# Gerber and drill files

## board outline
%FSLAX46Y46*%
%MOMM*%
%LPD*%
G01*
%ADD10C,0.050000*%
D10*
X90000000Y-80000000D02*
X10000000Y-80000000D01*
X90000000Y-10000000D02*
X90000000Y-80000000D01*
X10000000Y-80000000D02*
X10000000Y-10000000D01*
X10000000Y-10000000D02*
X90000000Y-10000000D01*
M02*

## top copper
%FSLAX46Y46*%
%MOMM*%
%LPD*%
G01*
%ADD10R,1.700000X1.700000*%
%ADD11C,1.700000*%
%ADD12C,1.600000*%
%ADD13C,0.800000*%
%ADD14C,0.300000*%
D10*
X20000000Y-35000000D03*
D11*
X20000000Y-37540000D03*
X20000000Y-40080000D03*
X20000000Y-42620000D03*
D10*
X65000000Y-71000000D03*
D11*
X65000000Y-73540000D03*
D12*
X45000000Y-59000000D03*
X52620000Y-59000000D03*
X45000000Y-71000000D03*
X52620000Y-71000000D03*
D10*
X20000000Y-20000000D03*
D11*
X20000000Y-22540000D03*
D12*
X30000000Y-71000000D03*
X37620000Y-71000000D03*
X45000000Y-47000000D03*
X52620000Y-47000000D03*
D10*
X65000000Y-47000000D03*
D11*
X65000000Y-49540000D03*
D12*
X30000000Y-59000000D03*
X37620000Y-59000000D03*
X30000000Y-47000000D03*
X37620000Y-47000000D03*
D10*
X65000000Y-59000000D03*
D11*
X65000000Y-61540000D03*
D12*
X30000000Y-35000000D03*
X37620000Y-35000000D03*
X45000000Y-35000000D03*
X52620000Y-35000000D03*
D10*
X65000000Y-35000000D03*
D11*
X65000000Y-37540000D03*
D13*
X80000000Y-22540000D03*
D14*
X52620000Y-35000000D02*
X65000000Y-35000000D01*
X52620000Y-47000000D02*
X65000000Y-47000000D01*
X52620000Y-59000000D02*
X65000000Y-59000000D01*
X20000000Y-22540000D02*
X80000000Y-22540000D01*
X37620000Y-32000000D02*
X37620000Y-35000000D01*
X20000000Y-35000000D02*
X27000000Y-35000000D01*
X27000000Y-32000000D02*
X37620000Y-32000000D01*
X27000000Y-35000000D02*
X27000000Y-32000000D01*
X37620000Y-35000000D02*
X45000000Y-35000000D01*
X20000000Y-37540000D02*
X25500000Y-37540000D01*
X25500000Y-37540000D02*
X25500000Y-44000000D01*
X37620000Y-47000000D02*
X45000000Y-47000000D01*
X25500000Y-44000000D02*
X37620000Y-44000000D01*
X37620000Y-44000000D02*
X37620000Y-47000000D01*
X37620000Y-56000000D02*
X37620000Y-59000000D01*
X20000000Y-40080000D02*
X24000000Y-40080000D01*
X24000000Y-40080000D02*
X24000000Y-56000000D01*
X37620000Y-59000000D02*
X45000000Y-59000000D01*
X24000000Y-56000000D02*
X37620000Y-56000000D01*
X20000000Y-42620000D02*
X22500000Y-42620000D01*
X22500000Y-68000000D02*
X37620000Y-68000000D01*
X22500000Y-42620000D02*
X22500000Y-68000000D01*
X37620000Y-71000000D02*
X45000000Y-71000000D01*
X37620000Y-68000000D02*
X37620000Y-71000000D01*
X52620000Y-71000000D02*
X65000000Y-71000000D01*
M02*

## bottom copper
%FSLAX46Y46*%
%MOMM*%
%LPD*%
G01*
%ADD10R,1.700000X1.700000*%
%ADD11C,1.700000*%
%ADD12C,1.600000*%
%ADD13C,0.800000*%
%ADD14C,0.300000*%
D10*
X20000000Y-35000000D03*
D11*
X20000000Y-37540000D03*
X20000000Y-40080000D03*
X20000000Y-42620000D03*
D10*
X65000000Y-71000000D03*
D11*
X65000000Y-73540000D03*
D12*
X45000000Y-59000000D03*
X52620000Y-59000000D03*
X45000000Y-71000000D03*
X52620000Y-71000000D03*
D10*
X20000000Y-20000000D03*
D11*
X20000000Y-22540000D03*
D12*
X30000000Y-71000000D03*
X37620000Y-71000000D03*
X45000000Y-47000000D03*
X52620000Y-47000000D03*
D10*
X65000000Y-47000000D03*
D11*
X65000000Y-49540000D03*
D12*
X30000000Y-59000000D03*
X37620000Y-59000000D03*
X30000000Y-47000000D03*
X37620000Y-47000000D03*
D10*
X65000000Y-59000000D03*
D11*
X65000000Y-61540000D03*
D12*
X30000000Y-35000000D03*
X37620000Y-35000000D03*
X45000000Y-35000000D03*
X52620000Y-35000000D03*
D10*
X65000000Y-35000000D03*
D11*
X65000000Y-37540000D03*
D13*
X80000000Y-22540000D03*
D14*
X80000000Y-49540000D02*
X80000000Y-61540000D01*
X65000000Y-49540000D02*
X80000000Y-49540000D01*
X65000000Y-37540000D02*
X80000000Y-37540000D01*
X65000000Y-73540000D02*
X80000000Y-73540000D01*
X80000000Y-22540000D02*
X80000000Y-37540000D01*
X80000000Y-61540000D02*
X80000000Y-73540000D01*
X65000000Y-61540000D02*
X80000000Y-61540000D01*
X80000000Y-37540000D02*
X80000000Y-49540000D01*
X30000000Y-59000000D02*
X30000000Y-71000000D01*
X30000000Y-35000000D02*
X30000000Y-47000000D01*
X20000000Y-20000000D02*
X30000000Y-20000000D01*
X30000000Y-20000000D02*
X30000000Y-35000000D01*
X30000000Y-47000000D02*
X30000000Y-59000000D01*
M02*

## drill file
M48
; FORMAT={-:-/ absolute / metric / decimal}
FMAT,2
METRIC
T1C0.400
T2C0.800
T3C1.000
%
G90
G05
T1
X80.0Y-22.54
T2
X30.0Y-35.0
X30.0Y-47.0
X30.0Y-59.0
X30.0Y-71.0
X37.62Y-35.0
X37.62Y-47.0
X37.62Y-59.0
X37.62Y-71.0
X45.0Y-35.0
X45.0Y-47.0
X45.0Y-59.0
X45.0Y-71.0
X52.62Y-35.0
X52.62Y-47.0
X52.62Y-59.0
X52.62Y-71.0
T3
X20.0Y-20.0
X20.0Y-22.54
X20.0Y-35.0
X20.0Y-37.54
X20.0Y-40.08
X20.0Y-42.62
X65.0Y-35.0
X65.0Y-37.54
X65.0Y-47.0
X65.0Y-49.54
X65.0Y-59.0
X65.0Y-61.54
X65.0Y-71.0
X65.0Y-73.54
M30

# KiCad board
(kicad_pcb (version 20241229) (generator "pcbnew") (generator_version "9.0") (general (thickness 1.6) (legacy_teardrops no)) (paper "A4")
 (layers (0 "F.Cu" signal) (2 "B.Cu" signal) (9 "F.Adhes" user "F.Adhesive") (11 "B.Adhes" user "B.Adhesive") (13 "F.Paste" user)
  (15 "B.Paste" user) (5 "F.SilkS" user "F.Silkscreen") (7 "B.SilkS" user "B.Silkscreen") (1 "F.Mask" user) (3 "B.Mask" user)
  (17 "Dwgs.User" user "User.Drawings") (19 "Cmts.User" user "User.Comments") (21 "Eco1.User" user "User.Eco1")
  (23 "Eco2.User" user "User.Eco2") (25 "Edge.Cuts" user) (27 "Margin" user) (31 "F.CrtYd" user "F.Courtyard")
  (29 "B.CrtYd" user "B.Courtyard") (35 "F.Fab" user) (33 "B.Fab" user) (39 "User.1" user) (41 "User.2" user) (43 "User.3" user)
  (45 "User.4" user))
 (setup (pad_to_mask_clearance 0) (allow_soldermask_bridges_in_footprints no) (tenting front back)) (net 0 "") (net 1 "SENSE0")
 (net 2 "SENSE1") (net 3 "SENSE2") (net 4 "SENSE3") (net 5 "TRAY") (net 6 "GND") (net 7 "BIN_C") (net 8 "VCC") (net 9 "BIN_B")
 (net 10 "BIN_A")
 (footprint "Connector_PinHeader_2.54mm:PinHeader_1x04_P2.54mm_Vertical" (layer "F.Cu") (at 20 35)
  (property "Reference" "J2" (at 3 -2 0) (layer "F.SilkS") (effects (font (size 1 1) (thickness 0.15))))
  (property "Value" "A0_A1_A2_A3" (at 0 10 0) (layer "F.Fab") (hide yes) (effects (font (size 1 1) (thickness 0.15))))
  (pad "1" thru_hole rect (at 0 0) (size 1.7 1.7) (drill 1) (layers "*.Cu" "*.Mask") (remove_unused_layers no) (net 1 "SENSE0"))
  (pad "2" thru_hole circle (at 0 2.54) (size 1.7 1.7) (drill 1) (layers "*.Cu" "*.Mask") (remove_unused_layers no) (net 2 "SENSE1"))
  (pad "3" thru_hole circle (at 0 5.08) (size 1.7 1.7) (drill 1) (layers "*.Cu" "*.Mask") (remove_unused_layers no) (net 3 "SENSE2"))
  (pad "4" thru_hole circle (at 0 7.62) (size 1.7 1.7) (drill 1) (layers "*.Cu" "*.Mask") (remove_unused_layers no) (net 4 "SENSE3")))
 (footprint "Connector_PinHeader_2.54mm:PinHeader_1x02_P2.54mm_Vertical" (layer "F.Cu") (at 65 71)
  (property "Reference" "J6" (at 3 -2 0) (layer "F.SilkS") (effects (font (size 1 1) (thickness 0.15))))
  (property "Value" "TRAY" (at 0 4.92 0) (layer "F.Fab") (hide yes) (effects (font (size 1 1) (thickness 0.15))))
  (pad "1" thru_hole rect (at 0 0) (size 1.7 1.7) (drill 1) (layers "*.Cu" "*.Mask") (remove_unused_layers no) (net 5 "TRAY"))
  (pad "2" thru_hole circle (at 0 2.54) (size 1.7 1.7) (drill 1) (layers "*.Cu" "*.Mask") (remove_unused_layers no) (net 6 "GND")))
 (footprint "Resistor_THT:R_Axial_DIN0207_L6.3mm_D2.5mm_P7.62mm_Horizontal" (layer "F.Cu") (at 45 59)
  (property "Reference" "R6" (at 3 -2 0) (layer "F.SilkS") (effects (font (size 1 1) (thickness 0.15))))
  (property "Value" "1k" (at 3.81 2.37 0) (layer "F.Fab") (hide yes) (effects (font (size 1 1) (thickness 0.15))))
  (pad "1" thru_hole circle (at 0 0) (size 1.6 1.6) (drill 0.8) (layers "*.Cu" "*.Mask") (remove_unused_layers no) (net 3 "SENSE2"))
  (pad "2" thru_hole circle (at 7.62 0) (size 1.6 1.6) (drill 0.8) (layers "*.Cu" "*.Mask") (remove_unused_layers no) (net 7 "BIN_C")))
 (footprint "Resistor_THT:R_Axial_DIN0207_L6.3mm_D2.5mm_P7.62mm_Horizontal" (layer "F.Cu") (at 45 71)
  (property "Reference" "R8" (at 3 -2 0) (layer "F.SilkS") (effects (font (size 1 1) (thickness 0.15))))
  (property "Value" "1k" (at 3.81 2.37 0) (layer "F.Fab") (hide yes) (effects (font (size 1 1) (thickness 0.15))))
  (pad "1" thru_hole circle (at 0 0) (size 1.6 1.6) (drill 0.8) (layers "*.Cu" "*.Mask") (remove_unused_layers no) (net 4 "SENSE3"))
  (pad "2" thru_hole circle (at 7.62 0) (size 1.6 1.6) (drill 0.8) (layers "*.Cu" "*.Mask") (remove_unused_layers no) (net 5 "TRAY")))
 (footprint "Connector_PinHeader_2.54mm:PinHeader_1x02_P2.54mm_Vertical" (layer "F.Cu") (at 20 20)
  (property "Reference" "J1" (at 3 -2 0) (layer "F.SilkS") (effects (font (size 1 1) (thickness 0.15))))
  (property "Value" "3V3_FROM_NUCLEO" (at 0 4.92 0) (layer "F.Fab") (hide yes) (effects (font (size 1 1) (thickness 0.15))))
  (pad "1" thru_hole rect (at 0 0) (size 1.7 1.7) (drill 1) (layers "*.Cu" "*.Mask") (remove_unused_layers no) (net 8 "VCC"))
  (pad "2" thru_hole circle (at 0 2.54) (size 1.7 1.7) (drill 1) (layers "*.Cu" "*.Mask") (remove_unused_layers no) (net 6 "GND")))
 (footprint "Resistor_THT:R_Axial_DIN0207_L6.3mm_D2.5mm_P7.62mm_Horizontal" (layer "F.Cu") (at 30 71)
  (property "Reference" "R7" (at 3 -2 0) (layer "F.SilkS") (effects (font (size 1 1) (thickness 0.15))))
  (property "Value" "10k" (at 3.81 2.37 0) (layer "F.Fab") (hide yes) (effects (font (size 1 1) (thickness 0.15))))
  (pad "1" thru_hole circle (at 0 0) (size 1.6 1.6) (drill 0.8) (layers "*.Cu" "*.Mask") (remove_unused_layers no) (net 8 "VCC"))
  (pad "2" thru_hole circle (at 7.62 0) (size 1.6 1.6) (drill 0.8) (layers "*.Cu" "*.Mask") (remove_unused_layers no) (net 4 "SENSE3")))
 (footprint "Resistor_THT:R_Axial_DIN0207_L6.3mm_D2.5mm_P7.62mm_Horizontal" (layer "F.Cu") (at 45 47)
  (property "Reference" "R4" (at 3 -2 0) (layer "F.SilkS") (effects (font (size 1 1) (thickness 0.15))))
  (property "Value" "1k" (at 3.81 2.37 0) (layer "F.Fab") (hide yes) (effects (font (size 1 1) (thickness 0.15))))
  (pad "1" thru_hole circle (at 0 0) (size 1.6 1.6) (drill 0.8) (layers "*.Cu" "*.Mask") (remove_unused_layers no) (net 2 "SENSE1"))
  (pad "2" thru_hole circle (at 7.62 0) (size 1.6 1.6) (drill 0.8) (layers "*.Cu" "*.Mask") (remove_unused_layers no) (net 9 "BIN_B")))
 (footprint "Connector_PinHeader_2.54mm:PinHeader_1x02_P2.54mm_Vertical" (layer "F.Cu") (at 65 47)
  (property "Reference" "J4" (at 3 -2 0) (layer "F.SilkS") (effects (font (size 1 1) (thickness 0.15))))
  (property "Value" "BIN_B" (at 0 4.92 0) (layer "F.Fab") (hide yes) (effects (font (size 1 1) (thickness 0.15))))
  (pad "1" thru_hole rect (at 0 0) (size 1.7 1.7) (drill 1) (layers "*.Cu" "*.Mask") (remove_unused_layers no) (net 9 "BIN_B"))
  (pad "2" thru_hole circle (at 0 2.54) (size 1.7 1.7) (drill 1) (layers "*.Cu" "*.Mask") (remove_unused_layers no) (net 6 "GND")))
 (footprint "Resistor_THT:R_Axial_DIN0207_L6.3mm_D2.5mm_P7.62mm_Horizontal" (layer "F.Cu") (at 30 59)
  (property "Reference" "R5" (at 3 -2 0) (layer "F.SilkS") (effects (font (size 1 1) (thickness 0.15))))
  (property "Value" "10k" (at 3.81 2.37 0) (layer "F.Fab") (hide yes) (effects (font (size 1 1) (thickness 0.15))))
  (pad "1" thru_hole circle (at 0 0) (size 1.6 1.6) (drill 0.8) (layers "*.Cu" "*.Mask") (remove_unused_layers no) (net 8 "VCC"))
  (pad "2" thru_hole circle (at 7.62 0) (size 1.6 1.6) (drill 0.8) (layers "*.Cu" "*.Mask") (remove_unused_layers no) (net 3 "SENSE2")))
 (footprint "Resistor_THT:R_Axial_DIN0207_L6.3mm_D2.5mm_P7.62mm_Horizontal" (layer "F.Cu") (at 30 47)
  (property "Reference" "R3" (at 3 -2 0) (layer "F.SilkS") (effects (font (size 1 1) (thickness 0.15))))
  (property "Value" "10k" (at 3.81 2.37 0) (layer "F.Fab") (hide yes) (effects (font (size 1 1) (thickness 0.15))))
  (pad "1" thru_hole circle (at 0 0) (size 1.6 1.6) (drill 0.8) (layers "*.Cu" "*.Mask") (remove_unused_layers no) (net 8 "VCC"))
  (pad "2" thru_hole circle (at 7.62 0) (size 1.6 1.6) (drill 0.8) (layers "*.Cu" "*.Mask") (remove_unused_layers no) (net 2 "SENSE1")))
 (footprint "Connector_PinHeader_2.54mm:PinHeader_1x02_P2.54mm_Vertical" (layer "F.Cu") (at 65 59)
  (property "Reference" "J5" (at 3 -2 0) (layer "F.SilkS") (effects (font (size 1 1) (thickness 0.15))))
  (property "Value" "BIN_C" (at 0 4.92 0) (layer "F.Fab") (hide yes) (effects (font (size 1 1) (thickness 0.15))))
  (pad "1" thru_hole rect (at 0 0) (size 1.7 1.7) (drill 1) (layers "*.Cu" "*.Mask") (remove_unused_layers no) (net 7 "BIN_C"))
  (pad "2" thru_hole circle (at 0 2.54) (size 1.7 1.7) (drill 1) (layers "*.Cu" "*.Mask") (remove_unused_layers no) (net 6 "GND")))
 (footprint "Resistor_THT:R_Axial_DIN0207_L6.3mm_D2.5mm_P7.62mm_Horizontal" (layer "F.Cu") (at 30 35)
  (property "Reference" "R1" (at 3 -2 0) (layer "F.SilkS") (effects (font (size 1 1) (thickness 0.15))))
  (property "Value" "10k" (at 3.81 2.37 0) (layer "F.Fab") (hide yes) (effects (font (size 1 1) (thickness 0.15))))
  (pad "1" thru_hole circle (at 0 0) (size 1.6 1.6) (drill 0.8) (layers "*.Cu" "*.Mask") (remove_unused_layers no) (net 8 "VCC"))
  (pad "2" thru_hole circle (at 7.62 0) (size 1.6 1.6) (drill 0.8) (layers "*.Cu" "*.Mask") (remove_unused_layers no) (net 1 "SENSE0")))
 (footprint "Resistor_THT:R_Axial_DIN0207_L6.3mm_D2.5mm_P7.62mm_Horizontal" (layer "F.Cu") (at 45 35)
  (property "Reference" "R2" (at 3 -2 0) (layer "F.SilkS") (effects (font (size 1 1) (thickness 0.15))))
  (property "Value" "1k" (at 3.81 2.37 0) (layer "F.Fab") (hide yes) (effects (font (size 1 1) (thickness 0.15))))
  (pad "1" thru_hole circle (at 0 0) (size 1.6 1.6) (drill 0.8) (layers "*.Cu" "*.Mask") (remove_unused_layers no) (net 1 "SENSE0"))
  (pad "2" thru_hole circle (at 7.62 0) (size 1.6 1.6) (drill 0.8) (layers "*.Cu" "*.Mask") (remove_unused_layers no) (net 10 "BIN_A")))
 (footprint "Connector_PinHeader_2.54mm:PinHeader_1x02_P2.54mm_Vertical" (layer "F.Cu") (at 65 35)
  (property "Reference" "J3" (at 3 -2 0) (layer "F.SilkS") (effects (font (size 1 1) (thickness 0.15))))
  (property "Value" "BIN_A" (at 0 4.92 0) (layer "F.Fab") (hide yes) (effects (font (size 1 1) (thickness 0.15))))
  (pad "1" thru_hole rect (at 0 0) (size 1.7 1.7) (drill 1) (layers "*.Cu" "*.Mask") (remove_unused_layers no) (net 10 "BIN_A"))
  (pad "2" thru_hole circle (at 0 2.54) (size 1.7 1.7) (drill 1) (layers "*.Cu" "*.Mask") (remove_unused_layers no) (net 6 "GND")))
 (gr_line (start 90 80) (end 10 80) (stroke (width 0.05) (type default)) (layer "Edge.Cuts"))
 (gr_line (start 90 10) (end 90 80) (stroke (width 0.05) (type default)) (layer "Edge.Cuts"))
 (gr_line (start 10 80) (end 10 10) (stroke (width 0.05) (type default)) (layer "Edge.Cuts"))
 (gr_line (start 10 10) (end 90 10) (stroke (width 0.05) (type default)) (layer "Edge.Cuts"))
 (segment (start 52.62 35) (end 65 35) (width 0.3) (layer "F.Cu") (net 10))
 (segment (start 52.62 47) (end 65 47) (width 0.3) (layer "F.Cu") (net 9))
 (segment (start 52.62 59) (end 65 59) (width 0.3) (layer "F.Cu") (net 7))
 (segment (start 20 22.54) (end 80 22.54) (width 0.3) (layer "F.Cu") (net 6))
 (via (at 80 22.54) (size 0.8) (drill 0.4) (layers "F.Cu" "B.Cu") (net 6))
 (segment (start 80 49.54) (end 80 61.54) (width 0.3) (layer "B.Cu") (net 6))
 (segment (start 65 49.54) (end 80 49.54) (width 0.3) (layer "B.Cu") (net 6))
 (segment (start 65 37.54) (end 80 37.54) (width 0.3) (layer "B.Cu") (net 6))
 (segment (start 65 73.54) (end 80 73.54) (width 0.3) (layer "B.Cu") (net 6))
 (segment (start 80 22.54) (end 80 37.54) (width 0.3) (layer "B.Cu") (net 6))
 (segment (start 80 61.54) (end 80 73.54) (width 0.3) (layer "B.Cu") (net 6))
 (segment (start 65 61.54) (end 80 61.54) (width 0.3) (layer "B.Cu") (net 6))
 (segment (start 80 37.54) (end 80 49.54) (width 0.3) (layer "B.Cu") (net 6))
 (segment (start 37.62 32) (end 37.62 35) (width 0.3) (layer "F.Cu") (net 1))
 (segment (start 20 35) (end 27 35) (width 0.3) (layer "F.Cu") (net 1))
 (segment (start 27 32) (end 37.62 32) (width 0.3) (layer "F.Cu") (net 1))
 (segment (start 27 35) (end 27 32) (width 0.3) (layer "F.Cu") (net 1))
 (segment (start 37.62 35) (end 45 35) (width 0.3) (layer "F.Cu") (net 1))
 (segment (start 20 37.54) (end 25.5 37.54) (width 0.3) (layer "F.Cu") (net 2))
 (segment (start 25.5 37.54) (end 25.5 44) (width 0.3) (layer "F.Cu") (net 2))
 (segment (start 37.62 47) (end 45 47) (width 0.3) (layer "F.Cu") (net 2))
 (segment (start 25.5 44) (end 37.62 44) (width 0.3) (layer "F.Cu") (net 2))
 (segment (start 37.62 44) (end 37.62 47) (width 0.3) (layer "F.Cu") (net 2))
 (segment (start 37.62 56) (end 37.62 59) (width 0.3) (layer "F.Cu") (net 3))
 (segment (start 20 40.08) (end 24 40.08) (width 0.3) (layer "F.Cu") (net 3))
 (segment (start 24 40.08) (end 24 56) (width 0.3) (layer "F.Cu") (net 3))
 (segment (start 37.62 59) (end 45 59) (width 0.3) (layer "F.Cu") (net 3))
 (segment (start 24 56) (end 37.62 56) (width 0.3) (layer "F.Cu") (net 3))
 (segment (start 20 42.62) (end 22.5 42.62) (width 0.3) (layer "F.Cu") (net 4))
 (segment (start 22.5 68) (end 37.62 68) (width 0.3) (layer "F.Cu") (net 4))
 (segment (start 22.5 42.62) (end 22.5 68) (width 0.3) (layer "F.Cu") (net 4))
 (segment (start 37.62 71) (end 45 71) (width 0.3) (layer "F.Cu") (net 4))
 (segment (start 37.62 68) (end 37.62 71) (width 0.3) (layer "F.Cu") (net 4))
 (segment (start 52.62 71) (end 65 71) (width 0.3) (layer "F.Cu") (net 5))
 (segment (start 30 59) (end 30 71) (width 0.3) (layer "B.Cu") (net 8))
 (segment (start 30 35) (end 30 47) (width 0.3) (layer "B.Cu") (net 8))
 (segment (start 20 20) (end 30 20) (width 0.3) (layer "B.Cu") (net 8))
 (segment (start 30 20) (end 30 35) (width 0.3) (layer "B.Cu") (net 8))
 (segment (start 30 47) (end 30 59) (width 0.3) (layer "B.Cu") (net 8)))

